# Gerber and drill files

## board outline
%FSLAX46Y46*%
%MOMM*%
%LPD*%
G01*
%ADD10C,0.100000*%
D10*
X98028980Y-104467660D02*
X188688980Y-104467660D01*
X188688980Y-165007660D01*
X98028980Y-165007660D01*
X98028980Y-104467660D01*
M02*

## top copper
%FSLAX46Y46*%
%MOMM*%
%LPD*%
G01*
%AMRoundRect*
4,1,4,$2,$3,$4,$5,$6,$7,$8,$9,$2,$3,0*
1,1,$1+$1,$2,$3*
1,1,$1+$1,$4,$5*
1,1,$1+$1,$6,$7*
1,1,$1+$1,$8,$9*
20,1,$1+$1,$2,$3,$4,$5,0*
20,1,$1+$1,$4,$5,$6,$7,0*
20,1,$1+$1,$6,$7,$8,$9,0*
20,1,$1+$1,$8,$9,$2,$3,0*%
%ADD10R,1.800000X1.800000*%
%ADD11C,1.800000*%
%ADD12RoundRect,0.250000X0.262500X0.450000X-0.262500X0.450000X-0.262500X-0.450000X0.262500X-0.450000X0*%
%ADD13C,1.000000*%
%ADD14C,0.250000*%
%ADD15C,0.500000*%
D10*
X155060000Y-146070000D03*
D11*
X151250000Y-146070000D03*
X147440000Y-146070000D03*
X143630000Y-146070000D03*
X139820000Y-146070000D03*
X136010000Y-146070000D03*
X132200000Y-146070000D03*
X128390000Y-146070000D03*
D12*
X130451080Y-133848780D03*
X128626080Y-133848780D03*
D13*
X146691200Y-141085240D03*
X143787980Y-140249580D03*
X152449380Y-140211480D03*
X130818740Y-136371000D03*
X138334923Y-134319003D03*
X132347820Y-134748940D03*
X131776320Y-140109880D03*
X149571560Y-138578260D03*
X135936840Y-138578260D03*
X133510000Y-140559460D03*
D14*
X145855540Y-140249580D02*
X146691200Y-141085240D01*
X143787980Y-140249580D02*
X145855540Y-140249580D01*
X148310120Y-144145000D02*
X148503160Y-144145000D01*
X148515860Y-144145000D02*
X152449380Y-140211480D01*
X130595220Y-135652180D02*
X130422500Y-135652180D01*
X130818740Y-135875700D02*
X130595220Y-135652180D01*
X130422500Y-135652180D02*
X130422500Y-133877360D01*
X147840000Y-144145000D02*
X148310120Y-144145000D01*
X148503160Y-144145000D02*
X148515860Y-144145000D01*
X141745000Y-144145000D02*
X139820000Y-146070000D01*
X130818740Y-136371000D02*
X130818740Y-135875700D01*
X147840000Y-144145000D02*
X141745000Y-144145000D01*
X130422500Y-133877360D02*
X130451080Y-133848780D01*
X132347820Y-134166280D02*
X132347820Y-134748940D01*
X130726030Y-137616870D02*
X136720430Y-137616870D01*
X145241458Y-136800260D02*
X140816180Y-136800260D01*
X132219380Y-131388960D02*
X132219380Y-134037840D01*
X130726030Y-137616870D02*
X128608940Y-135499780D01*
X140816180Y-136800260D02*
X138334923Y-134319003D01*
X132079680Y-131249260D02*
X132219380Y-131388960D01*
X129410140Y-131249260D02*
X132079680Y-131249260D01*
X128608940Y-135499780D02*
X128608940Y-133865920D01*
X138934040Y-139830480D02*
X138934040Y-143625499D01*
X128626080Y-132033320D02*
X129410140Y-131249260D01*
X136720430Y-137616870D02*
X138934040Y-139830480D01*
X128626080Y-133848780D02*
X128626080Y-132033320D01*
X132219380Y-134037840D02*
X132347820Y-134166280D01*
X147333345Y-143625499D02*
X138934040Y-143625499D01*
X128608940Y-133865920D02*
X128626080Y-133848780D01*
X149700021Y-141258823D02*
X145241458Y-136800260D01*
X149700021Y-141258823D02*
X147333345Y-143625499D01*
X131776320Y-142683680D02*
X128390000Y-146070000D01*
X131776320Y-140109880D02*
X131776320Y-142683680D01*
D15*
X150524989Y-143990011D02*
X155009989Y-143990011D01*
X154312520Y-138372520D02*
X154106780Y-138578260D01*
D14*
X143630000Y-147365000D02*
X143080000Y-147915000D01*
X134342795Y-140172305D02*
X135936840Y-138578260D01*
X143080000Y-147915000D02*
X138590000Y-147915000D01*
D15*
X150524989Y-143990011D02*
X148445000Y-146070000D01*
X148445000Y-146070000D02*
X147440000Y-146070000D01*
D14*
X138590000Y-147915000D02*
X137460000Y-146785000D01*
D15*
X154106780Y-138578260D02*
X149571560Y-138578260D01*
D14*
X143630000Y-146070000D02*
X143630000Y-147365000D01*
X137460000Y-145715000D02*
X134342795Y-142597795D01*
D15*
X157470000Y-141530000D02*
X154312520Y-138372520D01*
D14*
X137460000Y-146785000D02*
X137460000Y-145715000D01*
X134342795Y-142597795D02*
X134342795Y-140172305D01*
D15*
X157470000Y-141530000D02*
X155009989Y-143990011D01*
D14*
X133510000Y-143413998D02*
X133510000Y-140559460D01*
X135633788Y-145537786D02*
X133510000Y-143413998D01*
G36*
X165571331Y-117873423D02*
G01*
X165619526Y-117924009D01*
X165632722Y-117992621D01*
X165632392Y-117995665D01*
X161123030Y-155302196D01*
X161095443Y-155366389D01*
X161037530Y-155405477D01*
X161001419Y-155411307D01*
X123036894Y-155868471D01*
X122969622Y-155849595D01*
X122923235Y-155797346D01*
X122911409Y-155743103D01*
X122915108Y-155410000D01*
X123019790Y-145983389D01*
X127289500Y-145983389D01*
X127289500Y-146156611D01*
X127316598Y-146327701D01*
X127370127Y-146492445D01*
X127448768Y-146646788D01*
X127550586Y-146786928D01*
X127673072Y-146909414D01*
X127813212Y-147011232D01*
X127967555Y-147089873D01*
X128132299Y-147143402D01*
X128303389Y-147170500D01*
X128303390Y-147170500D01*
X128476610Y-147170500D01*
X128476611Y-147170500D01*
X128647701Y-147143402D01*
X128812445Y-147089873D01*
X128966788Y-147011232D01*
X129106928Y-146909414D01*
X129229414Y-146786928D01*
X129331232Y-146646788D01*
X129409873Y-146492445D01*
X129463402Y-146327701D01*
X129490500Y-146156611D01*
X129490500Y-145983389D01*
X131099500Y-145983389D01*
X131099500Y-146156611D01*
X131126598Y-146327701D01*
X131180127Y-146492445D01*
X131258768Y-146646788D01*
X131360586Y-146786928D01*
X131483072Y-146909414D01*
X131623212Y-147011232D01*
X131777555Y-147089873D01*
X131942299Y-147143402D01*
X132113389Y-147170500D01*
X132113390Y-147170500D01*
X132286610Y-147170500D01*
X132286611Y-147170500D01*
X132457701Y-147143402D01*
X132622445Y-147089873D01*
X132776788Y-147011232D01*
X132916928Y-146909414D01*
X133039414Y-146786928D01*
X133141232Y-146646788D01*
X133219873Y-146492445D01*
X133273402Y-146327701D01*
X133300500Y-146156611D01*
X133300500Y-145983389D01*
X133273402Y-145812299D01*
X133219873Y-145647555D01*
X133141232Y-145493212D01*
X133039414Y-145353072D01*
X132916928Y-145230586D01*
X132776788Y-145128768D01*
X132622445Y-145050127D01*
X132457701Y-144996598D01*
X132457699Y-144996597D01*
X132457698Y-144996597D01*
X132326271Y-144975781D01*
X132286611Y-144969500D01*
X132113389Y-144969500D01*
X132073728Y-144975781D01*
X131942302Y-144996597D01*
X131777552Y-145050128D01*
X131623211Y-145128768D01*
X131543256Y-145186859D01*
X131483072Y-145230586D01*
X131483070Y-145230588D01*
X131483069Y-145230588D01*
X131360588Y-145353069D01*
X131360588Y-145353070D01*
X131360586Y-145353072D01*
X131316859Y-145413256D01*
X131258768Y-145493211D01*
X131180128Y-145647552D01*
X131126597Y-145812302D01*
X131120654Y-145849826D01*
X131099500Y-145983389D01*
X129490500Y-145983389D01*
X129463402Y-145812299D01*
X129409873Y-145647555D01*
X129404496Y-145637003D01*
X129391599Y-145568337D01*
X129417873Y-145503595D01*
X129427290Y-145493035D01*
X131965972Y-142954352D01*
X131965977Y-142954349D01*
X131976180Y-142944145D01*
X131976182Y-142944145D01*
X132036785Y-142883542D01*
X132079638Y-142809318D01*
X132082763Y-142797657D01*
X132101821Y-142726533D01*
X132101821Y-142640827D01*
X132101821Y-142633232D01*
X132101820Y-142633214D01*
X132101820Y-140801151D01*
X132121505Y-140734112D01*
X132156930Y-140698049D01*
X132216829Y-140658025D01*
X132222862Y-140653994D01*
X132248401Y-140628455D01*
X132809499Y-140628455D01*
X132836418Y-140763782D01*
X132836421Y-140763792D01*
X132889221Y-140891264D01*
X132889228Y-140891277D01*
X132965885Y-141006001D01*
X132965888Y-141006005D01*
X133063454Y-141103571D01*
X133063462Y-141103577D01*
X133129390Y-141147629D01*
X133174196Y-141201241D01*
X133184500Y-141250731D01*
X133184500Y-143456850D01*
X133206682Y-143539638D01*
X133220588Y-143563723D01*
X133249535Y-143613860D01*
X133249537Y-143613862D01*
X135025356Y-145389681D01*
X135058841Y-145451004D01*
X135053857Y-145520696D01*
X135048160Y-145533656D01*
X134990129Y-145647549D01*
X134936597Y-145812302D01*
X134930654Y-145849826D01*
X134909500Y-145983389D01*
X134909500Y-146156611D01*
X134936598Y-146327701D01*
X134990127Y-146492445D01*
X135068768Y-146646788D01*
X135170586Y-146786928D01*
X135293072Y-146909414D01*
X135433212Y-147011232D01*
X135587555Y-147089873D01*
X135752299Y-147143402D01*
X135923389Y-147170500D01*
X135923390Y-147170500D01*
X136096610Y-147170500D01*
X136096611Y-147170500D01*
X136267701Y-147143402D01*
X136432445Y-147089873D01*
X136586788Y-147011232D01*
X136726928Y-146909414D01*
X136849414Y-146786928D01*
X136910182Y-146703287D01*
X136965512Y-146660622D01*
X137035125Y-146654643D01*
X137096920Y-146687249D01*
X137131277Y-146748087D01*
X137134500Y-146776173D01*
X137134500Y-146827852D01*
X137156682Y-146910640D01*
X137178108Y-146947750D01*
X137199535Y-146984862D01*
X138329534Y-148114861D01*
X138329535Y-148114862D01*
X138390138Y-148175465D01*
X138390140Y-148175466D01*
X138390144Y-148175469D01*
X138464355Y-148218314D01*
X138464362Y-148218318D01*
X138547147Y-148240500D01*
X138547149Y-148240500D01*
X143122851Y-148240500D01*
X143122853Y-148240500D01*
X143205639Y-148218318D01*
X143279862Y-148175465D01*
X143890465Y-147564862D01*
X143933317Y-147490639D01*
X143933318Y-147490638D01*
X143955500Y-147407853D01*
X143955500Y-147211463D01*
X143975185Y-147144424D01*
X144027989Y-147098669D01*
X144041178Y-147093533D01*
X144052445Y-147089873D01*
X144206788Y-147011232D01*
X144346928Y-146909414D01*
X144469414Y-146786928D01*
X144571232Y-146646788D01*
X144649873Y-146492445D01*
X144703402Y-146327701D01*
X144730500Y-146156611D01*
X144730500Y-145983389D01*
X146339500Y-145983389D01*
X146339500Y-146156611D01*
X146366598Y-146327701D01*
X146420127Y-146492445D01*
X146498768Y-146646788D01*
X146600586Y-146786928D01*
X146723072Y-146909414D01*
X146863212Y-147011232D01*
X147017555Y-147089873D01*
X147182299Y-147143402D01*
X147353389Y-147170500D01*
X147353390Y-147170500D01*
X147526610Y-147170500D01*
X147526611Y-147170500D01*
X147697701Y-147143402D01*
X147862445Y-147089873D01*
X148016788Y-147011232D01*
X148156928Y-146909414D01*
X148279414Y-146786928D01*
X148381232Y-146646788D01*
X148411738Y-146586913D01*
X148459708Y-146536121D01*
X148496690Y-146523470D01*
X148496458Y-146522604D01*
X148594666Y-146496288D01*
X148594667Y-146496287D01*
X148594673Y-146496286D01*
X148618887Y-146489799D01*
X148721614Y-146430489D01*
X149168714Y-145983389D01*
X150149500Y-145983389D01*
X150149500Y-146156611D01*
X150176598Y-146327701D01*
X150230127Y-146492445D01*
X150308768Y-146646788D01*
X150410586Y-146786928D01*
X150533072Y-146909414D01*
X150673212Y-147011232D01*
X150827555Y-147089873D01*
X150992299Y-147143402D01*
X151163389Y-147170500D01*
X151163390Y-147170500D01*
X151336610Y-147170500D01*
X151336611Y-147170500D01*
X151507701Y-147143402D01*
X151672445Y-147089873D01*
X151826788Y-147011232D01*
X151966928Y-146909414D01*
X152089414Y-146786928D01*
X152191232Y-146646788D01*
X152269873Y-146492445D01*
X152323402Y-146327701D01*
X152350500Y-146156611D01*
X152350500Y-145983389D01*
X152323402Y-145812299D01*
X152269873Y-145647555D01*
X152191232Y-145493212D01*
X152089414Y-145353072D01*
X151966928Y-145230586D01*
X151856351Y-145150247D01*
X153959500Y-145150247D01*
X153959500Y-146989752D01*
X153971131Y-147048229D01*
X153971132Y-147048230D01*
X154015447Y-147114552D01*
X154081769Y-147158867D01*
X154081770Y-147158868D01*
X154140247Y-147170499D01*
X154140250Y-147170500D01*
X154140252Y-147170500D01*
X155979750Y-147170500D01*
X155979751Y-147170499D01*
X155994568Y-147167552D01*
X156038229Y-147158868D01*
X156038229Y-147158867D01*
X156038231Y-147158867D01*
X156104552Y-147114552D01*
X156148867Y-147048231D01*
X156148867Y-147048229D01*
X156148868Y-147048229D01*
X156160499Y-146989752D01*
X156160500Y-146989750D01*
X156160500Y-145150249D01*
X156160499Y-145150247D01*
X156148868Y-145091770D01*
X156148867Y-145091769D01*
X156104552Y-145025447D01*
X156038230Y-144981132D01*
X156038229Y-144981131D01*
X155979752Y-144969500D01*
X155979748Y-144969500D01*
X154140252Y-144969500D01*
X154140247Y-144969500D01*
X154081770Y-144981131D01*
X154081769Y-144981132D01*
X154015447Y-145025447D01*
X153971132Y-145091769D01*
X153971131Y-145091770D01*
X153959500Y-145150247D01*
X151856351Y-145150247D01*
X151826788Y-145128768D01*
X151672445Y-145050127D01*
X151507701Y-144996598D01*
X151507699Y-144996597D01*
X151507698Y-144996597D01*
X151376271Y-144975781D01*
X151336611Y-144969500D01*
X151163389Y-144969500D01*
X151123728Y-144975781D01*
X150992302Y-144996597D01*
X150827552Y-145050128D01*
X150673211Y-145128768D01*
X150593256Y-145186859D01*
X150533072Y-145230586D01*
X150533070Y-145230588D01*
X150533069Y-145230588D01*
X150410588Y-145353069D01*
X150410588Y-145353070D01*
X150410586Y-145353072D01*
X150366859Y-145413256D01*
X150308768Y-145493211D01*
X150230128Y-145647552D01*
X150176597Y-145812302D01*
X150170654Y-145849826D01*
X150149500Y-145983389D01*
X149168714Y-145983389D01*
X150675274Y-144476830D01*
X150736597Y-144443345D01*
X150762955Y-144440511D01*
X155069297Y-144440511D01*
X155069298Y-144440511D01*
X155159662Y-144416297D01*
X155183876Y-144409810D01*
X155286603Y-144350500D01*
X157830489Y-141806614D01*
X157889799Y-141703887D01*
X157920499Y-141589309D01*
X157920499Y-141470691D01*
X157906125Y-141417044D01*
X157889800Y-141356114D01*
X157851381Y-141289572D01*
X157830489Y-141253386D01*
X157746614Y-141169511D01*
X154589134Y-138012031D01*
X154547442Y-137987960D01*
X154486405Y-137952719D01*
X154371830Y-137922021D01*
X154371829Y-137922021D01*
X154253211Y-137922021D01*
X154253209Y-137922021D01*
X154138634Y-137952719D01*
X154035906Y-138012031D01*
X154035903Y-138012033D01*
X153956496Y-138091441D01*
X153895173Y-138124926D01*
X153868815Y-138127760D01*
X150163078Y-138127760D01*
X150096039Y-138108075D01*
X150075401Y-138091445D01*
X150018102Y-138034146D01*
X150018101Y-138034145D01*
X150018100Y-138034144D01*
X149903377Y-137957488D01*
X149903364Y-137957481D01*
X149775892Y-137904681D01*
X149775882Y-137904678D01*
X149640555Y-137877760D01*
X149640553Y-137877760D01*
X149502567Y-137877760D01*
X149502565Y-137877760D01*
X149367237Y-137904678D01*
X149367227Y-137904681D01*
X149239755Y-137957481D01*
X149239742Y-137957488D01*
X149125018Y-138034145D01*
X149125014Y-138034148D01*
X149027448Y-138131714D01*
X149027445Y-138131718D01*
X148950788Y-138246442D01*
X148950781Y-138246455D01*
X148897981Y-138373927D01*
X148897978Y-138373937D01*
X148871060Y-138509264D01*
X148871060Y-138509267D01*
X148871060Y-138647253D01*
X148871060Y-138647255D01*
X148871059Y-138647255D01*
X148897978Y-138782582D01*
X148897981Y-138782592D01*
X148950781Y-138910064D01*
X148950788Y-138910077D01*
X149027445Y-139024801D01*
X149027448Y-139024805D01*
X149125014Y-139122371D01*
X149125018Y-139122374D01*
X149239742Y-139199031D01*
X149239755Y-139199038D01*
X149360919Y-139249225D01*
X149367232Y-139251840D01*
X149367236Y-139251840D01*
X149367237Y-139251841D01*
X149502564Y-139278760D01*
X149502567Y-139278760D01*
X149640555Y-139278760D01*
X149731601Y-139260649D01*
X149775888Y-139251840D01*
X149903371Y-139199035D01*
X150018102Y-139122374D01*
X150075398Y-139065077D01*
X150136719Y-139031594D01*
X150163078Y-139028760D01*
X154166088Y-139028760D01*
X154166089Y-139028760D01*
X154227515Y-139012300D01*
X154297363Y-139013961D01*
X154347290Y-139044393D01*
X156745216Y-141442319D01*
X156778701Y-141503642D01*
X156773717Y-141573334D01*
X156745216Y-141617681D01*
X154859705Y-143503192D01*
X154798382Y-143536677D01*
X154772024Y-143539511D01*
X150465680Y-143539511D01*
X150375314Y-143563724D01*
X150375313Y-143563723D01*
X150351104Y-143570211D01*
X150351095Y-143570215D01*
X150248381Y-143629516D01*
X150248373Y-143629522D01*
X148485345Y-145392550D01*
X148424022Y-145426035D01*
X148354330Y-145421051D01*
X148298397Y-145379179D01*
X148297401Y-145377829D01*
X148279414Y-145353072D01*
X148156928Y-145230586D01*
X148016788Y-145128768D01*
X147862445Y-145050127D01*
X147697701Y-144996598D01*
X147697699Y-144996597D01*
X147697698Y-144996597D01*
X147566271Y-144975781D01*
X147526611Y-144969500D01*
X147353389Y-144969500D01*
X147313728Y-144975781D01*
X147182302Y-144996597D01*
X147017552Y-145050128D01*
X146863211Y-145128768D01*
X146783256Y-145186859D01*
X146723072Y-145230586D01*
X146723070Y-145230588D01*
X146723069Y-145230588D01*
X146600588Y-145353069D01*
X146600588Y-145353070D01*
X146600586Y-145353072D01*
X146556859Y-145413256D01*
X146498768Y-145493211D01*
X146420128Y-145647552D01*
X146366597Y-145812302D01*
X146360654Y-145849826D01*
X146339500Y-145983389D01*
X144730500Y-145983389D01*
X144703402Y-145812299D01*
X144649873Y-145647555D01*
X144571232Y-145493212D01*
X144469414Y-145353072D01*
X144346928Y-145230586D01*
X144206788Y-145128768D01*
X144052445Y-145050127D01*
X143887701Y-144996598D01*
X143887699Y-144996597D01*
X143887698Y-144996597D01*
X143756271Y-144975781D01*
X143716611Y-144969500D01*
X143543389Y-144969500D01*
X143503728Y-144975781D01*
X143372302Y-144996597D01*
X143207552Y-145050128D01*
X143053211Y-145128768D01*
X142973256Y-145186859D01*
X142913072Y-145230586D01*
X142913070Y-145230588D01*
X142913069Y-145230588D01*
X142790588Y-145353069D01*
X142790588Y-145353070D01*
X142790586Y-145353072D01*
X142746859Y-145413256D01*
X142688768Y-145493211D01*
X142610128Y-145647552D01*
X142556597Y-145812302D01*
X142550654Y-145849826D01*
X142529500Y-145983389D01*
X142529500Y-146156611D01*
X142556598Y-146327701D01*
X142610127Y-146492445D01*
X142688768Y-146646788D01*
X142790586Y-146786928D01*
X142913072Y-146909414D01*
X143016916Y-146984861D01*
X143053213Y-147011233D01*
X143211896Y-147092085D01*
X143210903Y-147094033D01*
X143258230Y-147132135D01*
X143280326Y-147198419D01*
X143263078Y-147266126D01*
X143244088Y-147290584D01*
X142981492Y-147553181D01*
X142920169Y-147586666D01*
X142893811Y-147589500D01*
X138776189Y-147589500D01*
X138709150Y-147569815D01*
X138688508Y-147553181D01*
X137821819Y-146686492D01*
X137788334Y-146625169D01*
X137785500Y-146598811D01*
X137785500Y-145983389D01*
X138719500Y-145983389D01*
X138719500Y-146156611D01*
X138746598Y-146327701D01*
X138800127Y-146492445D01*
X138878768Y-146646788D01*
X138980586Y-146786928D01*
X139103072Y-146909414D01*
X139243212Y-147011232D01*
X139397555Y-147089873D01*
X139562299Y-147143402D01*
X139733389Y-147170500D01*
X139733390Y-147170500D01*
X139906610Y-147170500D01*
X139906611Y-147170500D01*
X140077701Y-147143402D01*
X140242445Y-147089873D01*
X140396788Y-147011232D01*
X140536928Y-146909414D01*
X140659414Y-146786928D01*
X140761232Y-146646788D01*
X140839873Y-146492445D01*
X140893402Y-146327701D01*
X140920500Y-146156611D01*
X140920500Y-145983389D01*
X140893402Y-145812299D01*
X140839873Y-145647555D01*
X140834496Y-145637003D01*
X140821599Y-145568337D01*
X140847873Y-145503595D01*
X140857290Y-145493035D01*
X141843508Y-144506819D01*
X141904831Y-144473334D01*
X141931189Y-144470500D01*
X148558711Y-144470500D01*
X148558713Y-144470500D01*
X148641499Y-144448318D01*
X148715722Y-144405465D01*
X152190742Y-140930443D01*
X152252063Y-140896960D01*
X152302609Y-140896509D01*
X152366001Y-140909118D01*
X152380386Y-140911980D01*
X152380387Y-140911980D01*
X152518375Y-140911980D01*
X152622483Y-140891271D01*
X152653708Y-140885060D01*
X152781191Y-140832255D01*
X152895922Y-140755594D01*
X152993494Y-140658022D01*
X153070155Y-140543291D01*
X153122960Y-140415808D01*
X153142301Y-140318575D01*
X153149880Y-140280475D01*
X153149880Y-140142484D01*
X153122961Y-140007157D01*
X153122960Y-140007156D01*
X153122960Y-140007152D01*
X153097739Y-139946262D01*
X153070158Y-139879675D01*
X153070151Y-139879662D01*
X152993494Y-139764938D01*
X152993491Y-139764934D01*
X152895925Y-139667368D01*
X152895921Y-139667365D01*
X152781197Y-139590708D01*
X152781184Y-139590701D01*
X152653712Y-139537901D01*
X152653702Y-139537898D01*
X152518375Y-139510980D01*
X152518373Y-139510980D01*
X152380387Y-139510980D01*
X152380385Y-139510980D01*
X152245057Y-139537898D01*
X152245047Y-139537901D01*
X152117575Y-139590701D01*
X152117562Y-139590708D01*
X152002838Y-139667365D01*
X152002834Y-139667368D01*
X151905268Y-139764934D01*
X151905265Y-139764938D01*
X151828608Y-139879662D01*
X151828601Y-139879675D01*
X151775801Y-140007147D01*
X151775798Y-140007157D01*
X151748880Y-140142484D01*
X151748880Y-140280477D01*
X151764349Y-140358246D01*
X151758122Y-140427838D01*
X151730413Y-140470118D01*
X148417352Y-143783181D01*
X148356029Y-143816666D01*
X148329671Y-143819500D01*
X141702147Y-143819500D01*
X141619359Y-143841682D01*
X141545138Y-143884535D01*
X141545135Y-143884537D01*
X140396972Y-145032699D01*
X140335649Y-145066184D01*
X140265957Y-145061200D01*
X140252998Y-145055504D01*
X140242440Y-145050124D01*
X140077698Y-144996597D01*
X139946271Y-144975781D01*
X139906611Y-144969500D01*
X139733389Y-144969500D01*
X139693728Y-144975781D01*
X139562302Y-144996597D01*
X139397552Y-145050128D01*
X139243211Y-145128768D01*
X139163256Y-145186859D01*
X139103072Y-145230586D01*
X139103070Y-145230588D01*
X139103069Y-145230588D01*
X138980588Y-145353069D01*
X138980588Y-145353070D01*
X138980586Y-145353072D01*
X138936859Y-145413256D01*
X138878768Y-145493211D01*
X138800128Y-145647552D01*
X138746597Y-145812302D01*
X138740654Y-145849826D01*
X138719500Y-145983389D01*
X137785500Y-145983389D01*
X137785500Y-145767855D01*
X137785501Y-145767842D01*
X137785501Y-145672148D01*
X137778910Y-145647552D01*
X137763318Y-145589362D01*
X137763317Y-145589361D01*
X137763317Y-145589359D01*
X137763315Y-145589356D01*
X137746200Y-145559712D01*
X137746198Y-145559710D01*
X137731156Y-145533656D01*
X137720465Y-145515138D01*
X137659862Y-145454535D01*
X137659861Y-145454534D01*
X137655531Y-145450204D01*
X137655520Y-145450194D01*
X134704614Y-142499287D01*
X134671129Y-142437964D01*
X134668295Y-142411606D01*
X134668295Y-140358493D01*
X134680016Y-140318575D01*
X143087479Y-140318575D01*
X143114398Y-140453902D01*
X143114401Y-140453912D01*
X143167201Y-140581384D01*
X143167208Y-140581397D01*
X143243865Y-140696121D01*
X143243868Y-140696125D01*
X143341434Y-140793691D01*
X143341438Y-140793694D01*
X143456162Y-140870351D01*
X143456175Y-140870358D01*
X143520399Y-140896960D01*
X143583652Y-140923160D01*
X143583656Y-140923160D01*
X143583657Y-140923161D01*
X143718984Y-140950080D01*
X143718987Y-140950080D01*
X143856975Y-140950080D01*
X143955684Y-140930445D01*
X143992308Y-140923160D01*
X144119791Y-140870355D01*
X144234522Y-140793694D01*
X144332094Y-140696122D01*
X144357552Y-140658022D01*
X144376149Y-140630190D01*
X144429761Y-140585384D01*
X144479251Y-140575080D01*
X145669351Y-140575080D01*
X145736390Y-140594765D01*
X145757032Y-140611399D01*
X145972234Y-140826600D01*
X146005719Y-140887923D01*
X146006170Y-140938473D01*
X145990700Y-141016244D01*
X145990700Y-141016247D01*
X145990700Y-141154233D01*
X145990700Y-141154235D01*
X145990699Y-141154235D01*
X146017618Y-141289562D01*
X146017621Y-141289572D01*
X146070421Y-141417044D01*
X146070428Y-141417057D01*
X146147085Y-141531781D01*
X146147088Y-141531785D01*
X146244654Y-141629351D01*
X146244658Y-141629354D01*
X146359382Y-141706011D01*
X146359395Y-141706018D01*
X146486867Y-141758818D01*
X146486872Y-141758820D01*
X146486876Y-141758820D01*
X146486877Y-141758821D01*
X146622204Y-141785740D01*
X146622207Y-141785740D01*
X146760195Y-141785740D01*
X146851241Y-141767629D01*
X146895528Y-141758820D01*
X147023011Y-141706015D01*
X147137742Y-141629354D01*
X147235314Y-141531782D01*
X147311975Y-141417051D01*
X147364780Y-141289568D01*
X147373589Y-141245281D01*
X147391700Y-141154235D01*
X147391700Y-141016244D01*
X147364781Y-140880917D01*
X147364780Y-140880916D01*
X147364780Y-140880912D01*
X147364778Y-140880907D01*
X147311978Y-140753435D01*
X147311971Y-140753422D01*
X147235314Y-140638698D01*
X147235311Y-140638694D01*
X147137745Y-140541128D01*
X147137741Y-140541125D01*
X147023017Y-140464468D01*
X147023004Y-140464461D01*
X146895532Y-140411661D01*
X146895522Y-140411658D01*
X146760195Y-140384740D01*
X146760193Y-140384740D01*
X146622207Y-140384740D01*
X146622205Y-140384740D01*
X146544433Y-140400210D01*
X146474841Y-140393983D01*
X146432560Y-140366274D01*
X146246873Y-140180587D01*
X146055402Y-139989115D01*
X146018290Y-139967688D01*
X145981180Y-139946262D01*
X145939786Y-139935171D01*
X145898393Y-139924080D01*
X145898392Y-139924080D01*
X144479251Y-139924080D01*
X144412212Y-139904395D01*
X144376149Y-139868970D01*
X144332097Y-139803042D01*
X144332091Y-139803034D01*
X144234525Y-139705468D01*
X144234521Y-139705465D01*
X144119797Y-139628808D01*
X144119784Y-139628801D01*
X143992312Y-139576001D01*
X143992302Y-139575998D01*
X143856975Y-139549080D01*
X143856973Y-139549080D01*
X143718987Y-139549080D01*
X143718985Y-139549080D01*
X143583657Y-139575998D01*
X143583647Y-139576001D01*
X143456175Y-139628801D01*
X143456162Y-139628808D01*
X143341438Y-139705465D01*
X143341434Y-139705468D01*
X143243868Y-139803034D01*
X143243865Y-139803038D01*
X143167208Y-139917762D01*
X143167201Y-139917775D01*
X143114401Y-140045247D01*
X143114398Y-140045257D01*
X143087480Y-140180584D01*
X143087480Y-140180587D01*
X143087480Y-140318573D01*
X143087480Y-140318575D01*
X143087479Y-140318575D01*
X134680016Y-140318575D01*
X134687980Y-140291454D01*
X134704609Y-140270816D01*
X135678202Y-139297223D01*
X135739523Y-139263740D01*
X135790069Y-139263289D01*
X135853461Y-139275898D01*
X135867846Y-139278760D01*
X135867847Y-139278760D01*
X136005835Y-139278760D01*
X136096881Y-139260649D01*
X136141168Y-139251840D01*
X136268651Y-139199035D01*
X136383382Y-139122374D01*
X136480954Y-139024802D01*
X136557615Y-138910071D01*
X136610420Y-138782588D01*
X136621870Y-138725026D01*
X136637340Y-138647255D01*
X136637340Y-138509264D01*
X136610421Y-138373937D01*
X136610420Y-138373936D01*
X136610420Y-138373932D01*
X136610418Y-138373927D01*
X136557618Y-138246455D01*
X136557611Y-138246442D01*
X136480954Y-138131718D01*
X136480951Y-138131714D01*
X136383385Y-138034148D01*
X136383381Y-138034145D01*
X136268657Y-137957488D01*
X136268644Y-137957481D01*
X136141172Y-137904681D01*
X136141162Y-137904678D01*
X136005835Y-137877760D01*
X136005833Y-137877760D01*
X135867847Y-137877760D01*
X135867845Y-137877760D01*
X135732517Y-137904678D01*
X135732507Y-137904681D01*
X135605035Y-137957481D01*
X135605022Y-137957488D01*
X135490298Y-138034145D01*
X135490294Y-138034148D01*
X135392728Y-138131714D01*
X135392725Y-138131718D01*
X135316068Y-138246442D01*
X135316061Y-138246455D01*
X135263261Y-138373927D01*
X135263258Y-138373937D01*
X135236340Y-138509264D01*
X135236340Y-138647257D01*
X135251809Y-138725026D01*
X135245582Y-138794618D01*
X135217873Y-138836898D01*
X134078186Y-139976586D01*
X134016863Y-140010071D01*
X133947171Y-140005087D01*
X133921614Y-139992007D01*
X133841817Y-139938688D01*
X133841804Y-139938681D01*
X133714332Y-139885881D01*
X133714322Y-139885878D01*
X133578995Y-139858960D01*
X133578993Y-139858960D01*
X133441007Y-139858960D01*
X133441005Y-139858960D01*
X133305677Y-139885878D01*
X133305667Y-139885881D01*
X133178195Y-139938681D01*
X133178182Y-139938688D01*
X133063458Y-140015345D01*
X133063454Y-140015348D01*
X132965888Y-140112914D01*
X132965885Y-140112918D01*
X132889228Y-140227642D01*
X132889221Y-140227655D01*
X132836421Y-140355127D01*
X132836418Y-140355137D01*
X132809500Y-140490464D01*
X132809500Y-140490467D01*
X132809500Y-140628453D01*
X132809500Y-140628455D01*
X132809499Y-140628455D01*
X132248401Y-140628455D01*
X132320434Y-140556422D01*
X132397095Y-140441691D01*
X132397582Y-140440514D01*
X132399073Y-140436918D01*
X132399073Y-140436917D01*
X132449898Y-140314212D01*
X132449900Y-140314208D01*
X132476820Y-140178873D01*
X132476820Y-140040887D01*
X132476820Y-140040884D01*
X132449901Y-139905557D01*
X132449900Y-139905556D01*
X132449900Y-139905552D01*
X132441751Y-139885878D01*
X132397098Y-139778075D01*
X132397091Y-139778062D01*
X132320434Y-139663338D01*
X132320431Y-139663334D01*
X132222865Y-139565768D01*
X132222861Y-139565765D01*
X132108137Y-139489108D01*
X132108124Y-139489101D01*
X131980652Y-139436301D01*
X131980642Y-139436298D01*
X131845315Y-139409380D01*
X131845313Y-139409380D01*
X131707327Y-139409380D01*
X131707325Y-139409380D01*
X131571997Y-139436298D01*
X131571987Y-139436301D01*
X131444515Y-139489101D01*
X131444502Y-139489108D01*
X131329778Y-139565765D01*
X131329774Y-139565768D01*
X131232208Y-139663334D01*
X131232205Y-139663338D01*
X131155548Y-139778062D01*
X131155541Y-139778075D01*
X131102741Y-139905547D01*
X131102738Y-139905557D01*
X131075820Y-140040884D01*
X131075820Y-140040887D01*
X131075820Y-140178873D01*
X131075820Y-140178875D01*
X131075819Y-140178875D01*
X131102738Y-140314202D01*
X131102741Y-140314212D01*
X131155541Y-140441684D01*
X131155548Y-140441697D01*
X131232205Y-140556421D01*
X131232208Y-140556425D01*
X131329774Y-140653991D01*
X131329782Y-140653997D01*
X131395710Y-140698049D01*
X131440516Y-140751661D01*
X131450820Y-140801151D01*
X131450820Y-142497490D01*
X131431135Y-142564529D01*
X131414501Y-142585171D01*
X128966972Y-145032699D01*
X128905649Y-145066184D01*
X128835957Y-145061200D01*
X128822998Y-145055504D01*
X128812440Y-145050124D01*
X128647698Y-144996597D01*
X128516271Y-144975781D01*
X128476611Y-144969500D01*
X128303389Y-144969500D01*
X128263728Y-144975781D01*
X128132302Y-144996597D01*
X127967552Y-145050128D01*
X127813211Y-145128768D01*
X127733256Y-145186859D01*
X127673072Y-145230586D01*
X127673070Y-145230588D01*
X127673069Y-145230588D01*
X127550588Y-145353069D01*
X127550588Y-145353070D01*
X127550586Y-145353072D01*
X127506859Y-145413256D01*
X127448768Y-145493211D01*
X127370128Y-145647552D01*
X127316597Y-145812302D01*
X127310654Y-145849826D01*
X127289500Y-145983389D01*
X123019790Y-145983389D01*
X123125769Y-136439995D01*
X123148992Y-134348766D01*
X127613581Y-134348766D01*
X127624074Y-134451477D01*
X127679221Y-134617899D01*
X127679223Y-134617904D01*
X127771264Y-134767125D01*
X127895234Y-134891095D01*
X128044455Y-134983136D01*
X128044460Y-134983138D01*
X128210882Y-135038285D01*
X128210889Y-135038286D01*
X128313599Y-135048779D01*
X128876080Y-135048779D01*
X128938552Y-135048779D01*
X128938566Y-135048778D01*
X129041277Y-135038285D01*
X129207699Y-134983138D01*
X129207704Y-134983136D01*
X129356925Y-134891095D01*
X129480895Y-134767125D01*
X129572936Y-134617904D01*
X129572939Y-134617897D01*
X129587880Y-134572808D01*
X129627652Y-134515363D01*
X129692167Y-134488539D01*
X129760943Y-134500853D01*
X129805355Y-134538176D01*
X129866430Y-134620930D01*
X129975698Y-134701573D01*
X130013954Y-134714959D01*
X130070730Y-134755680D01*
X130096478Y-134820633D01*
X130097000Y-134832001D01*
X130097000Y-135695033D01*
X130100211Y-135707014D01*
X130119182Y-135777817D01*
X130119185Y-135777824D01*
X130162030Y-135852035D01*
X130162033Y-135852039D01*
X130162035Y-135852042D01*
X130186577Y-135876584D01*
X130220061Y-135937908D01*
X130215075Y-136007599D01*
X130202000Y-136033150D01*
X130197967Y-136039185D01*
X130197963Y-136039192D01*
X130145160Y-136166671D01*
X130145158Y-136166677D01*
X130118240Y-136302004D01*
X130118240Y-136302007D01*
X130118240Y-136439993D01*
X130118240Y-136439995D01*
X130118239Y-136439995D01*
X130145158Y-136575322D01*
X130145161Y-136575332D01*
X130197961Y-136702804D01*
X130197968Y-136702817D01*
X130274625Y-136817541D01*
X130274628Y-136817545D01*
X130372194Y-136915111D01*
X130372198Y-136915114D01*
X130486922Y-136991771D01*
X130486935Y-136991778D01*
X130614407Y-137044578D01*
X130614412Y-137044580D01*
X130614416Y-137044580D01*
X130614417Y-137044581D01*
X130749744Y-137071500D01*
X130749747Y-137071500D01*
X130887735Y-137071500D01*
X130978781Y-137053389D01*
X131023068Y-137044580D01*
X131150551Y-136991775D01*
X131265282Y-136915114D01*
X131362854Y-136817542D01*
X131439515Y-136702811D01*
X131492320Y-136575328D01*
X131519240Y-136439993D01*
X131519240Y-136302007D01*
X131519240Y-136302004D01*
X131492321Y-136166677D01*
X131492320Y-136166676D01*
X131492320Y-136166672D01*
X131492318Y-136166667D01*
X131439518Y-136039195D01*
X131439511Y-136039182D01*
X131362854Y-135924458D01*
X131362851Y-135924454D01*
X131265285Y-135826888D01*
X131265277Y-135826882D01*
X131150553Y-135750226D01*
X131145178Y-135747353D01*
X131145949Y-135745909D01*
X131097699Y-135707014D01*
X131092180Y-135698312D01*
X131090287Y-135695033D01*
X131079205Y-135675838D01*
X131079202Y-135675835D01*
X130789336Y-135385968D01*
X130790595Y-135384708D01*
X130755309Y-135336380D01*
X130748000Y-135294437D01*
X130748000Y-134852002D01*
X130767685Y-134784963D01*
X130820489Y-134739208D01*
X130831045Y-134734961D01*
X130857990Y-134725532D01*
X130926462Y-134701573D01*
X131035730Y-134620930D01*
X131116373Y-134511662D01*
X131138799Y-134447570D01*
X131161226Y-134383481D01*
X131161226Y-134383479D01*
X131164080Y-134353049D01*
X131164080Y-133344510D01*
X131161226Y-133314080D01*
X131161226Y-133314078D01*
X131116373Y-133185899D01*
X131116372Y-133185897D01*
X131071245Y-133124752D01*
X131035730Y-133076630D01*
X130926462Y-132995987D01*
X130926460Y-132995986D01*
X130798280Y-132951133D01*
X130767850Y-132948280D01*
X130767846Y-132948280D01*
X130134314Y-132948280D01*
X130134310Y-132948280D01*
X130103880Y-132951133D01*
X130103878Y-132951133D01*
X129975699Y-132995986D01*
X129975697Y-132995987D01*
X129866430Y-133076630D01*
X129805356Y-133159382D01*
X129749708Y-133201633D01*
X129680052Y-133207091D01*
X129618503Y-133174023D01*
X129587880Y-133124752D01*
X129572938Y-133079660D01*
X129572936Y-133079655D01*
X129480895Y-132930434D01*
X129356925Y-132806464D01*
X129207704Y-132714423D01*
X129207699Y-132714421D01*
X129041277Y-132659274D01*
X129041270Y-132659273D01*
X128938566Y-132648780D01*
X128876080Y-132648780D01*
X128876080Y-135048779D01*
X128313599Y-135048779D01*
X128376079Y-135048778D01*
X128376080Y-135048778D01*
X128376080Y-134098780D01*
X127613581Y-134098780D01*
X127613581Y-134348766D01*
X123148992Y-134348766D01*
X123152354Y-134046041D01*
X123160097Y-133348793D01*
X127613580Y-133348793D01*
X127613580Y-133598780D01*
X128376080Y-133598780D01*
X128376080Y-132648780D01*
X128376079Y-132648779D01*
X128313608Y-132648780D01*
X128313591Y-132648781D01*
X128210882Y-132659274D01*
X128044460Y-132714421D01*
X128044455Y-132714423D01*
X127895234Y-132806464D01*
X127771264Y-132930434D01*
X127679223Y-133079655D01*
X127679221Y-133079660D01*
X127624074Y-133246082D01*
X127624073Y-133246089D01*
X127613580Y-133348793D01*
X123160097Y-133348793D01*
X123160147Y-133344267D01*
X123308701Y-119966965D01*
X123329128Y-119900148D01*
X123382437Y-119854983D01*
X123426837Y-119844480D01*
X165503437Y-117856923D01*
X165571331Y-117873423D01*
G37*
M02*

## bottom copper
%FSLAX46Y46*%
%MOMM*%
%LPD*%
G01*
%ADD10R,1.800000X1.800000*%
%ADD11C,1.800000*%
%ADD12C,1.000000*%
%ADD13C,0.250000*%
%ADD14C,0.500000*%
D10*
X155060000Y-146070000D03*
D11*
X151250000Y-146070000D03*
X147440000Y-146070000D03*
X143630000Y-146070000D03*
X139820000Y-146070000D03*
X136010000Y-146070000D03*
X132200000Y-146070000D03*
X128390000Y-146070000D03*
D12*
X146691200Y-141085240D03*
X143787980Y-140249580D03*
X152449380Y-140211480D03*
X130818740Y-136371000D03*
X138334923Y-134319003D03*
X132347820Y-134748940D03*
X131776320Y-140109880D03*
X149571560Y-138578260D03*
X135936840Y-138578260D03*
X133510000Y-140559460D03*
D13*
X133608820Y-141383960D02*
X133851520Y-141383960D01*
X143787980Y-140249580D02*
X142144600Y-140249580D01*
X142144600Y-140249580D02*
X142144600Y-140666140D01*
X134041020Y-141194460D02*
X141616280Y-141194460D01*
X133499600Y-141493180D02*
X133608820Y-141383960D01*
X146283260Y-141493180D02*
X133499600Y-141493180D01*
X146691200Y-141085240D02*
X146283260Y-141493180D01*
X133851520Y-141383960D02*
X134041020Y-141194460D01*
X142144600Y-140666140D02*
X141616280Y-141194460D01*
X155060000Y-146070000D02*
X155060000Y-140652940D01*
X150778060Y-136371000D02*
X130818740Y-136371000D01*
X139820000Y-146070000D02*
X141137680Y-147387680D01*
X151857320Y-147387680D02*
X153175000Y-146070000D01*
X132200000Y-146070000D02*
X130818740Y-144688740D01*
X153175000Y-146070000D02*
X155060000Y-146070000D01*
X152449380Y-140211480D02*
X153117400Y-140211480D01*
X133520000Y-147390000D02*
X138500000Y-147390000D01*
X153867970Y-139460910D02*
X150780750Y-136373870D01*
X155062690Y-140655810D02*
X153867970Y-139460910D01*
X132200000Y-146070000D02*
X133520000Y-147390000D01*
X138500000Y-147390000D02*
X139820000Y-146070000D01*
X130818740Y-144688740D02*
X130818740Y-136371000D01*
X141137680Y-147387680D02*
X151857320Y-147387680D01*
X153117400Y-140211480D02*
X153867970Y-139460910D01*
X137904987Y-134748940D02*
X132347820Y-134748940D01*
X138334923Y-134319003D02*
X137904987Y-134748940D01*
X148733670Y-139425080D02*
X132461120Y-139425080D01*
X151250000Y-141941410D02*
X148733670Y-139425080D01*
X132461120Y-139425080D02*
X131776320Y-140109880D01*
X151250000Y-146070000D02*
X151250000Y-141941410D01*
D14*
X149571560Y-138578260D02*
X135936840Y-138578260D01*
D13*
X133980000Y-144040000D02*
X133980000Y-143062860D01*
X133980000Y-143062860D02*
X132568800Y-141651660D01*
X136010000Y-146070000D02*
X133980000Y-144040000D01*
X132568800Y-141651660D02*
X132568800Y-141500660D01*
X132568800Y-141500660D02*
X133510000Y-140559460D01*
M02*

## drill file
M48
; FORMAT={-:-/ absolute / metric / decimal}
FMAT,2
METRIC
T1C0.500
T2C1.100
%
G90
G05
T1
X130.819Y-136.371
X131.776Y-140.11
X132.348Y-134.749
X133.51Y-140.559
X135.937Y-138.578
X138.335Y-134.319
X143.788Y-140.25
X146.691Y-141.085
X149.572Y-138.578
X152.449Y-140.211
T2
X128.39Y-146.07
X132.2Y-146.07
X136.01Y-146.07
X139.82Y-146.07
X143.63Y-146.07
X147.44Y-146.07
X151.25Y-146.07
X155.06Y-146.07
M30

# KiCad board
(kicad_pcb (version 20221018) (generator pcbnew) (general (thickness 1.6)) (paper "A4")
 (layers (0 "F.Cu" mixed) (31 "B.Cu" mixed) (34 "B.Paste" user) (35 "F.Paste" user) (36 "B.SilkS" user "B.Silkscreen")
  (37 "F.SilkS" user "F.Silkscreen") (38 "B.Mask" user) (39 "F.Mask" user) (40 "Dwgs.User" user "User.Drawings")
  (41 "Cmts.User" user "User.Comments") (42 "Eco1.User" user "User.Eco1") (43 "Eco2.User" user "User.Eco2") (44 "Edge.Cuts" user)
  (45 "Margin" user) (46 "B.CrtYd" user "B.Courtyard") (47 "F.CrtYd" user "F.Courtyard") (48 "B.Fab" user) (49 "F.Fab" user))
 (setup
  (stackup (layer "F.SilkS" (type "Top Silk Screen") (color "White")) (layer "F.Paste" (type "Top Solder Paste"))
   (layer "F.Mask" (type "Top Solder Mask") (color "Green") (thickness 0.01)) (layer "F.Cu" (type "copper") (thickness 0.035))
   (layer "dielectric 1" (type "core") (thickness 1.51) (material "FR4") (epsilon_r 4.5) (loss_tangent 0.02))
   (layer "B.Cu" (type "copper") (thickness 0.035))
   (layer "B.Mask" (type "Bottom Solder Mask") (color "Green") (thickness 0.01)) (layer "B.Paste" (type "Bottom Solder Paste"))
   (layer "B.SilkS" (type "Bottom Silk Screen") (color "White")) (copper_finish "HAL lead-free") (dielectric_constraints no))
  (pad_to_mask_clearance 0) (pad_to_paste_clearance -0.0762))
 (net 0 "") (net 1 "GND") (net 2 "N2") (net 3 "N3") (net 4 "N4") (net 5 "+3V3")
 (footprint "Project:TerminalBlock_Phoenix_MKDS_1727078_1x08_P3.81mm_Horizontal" (layer "F.Cu") (at 155.06 146.07 180)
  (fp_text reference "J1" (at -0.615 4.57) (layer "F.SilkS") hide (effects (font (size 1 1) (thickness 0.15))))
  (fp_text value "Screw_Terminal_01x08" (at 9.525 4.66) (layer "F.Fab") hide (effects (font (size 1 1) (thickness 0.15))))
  (pad "1" thru_hole rect (at 0 0 180) (size 1.8 1.8) (drill 1.1) (layers "*.Cu" "*.Mask") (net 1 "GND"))
  (pad "2" thru_hole circle (at 3.81 0 180) (size 1.8 1.8) (drill 1.1) (layers "*.Cu" "*.Mask") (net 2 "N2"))
  (pad "3" thru_hole circle (at 7.62 0 180) (size 1.8 1.8) (drill 1.1) (layers "*.Cu" "*.Mask") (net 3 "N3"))
  (pad "4" thru_hole circle (at 11.43 0 180) (size 1.8 1.8) (drill 1.1) (layers "*.Cu" "*.Mask") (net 3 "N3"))
  (pad "5" thru_hole circle (at 15.24 0 180) (size 1.8 1.8) (drill 1.1) (layers "*.Cu" "*.Mask") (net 1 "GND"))
  (pad "6" thru_hole circle (at 19.05 0 270) (size 1.8 1.8) (drill 1.1) (layers "*.Cu" "*.Mask") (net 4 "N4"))
  (pad "7" thru_hole circle (at 22.86 0 180) (size 1.8 1.8) (drill 1.1) (layers "*.Cu" "*.Mask") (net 1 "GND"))
  (pad "8" thru_hole circle (at 26.67 0 270) (size 1.8 1.8) (drill 1.1) (layers "*.Cu" "*.Mask") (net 2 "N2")))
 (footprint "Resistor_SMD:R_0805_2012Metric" (layer "F.Cu") (at 129.53858 133.84878 180)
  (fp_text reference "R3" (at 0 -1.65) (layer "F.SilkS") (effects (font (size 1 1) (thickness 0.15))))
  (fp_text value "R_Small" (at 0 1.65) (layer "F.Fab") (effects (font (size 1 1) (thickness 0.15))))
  (pad "1" smd roundrect (at -0.9125 0 180) (size 1.025 1.4) (layers "F.Cu" "F.Paste" "F.Mask") (roundrect_rratio 0.243902) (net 1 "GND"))
  (pad "2" smd roundrect (at 0.9125 0 180) (size 1.025 1.4) (layers "F.Cu" "F.Paste" "F.Mask") (roundrect_rratio 0.243902) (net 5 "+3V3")))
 (gr_rect (start 98.02898 104.46766) (end 188.68898 165.00766) (stroke (width 0.1) (type solid)) (fill none) (layer "Edge.Cuts"))
 (segment (start 145.85554 140.24958) (end 146.6912 141.08524) (width 0.25) (layer "F.Cu") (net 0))
 (segment (start 143.78798 140.24958) (end 145.85554 140.24958) (width 0.25) (layer "F.Cu") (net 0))
 (via (at 146.6912 141.08524) (size 1) (drill 0.5) (layers "F.Cu" "B.Cu") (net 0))
 (via (at 143.78798 140.24958) (size 1) (drill 0.5) (layers "F.Cu" "B.Cu") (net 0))
 (segment (start 133.60882 141.38396) (end 133.85152 141.38396) (width 0.25) (layer "B.Cu") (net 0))
 (segment locked (start 143.78798 140.24958) (end 142.1446 140.24958) (width 0.25) (layer "B.Cu") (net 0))
 (segment (start 142.1446 140.24958) (end 142.1446 140.66614) (width 0.25) (layer "B.Cu") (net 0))
 (segment (start 134.04102 141.19446) (end 141.61628 141.19446) (width 0.25) (layer "B.Cu") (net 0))
 (segment (start 133.4996 141.49318) (end 133.60882 141.38396) (width 0.25) (layer "B.Cu") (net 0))
 (segment (start 146.28326 141.49318) (end 133.4996 141.49318) (width 0.25) (layer "B.Cu") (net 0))
 (segment (start 146.6912 141.08524) (end 146.28326 141.49318) (width 0.25) (layer "B.Cu") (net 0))
 (segment (start 133.85152 141.38396) (end 134.04102 141.19446) (width 0.25) (layer "B.Cu") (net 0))
 (segment (start 142.1446 140.66614) (end 141.61628 141.19446) (width 0.25) (layer "B.Cu") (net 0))
 (segment (start 148.31012 144.145) (end 148.50316 144.145) (width 0.25) (layer "F.Cu") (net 1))
 (segment (start 148.51586 144.145) (end 152.44938 140.21148) (width 0.25) (layer "F.Cu") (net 1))
 (segment (start 130.59522 135.65218) (end 130.4225 135.65218) (width 0.25) (layer "F.Cu") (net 1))
 (segment (start 130.81874 135.8757) (end 130.59522 135.65218) (width 0.25) (layer "F.Cu") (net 1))
 (segment (start 130.4225 135.65218) (end 130.4225 133.87736) (width 0.25) (layer "F.Cu") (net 1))
 (segment (start 147.84 144.145) (end 148.31012 144.145) (width 0.25) (layer "F.Cu") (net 1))
 (segment (start 148.50316 144.145) (end 148.51586 144.145) (width 0.25) (layer "F.Cu") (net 1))
 (segment (start 141.745 144.145) (end 139.82 146.07) (width 0.25) (layer "F.Cu") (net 1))
 (segment (start 130.81874 136.371) (end 130.81874 135.8757) (width 0.25) (layer "F.Cu") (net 1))
 (segment (start 147.84 144.145) (end 141.745 144.145) (width 0.25) (layer "F.Cu") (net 1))
 (segment (start 130.4225 133.87736) (end 130.45108 133.84878) (width 0.25) (layer "F.Cu") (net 1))
 (via (at 152.44938 140.21148) (size 1) (drill 0.5) (layers "F.Cu" "B.Cu") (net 1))
 (via (at 130.81874 136.371) (size 1) (drill 0.5) (layers "F.Cu" "B.Cu") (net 1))
 (segment (start 155.06 146.07) (end 155.06 140.65294) (width 0.25) (layer "B.Cu") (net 1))
 (segment (start 150.77806 136.371) (end 130.81874 136.371) (width 0.25) (layer "B.Cu") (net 1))
 (segment (start 139.82 146.07) (end 141.13768 147.38768) (width 0.25) (layer "B.Cu") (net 1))
 (segment (start 151.85732 147.38768) (end 153.175 146.07) (width 0.25) (layer "B.Cu") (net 1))
 (segment (start 132.2 146.07) (end 130.81874 144.68874) (width 0.25) (layer "B.Cu") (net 1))
 (segment (start 153.175 146.07) (end 155.06 146.07) (width 0.25) (layer "B.Cu") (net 1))
 (segment (start 152.44938 140.21148) (end 153.1174 140.21148) (width 0.25) (layer "B.Cu") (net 1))
 (segment (start 133.52 147.39) (end 138.5 147.39) (width 0.25) (layer "B.Cu") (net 1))
 (segment (start 153.86797 139.46091) (end 150.78075 136.37387) (width 0.25) (layer "B.Cu") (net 1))
 (segment (start 155.06269 140.65581) (end 153.86797 139.46091) (width 0.25) (layer "B.Cu") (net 1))
 (segment (start 132.2 146.07) (end 133.52 147.39) (width 0.25) (layer "B.Cu") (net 1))
 (segment (start 138.5 147.39) (end 139.82 146.07) (width 0.25) (layer "B.Cu") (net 1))
 (segment (start 130.81874 144.68874) (end 130.81874 136.371) (width 0.25) (layer "B.Cu") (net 1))
 (segment (start 141.13768 147.38768) (end 151.85732 147.38768) (width 0.25) (layer "B.Cu") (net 1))
 (segment (start 153.1174 140.21148) (end 153.86797 139.46091) (width 0.25) (layer "B.Cu") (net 1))
 (segment (start 132.34782 134.16628) (end 132.34782 134.74894) (width 0.25) (layer "F.Cu") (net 5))
 (segment (start 130.72603 137.61687) (end 136.72043 137.61687) (width 0.25) (layer "F.Cu") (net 5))
 (segment (start 145.241458 136.80026) (end 140.81618 136.80026) (width 0.25) (layer "F.Cu") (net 5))
 (segment (start 132.21938 131.38896) (end 132.21938 134.03784) (width 0.25) (layer "F.Cu") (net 5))
 (segment (start 130.72603 137.61687) (end 128.60894 135.49978) (width 0.25) (layer "F.Cu") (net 5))
 (segment (start 140.81618 136.80026) (end 138.334923 134.319003) (width 0.25) (layer "F.Cu") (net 5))
 (segment (start 132.07968 131.24926) (end 132.21938 131.38896) (width 0.25) (layer "F.Cu") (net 5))
 (segment (start 129.41014 131.24926) (end 132.07968 131.24926) (width 0.25) (layer "F.Cu") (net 5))
 (segment (start 128.60894 135.49978) (end 128.60894 133.86592) (width 0.25) (layer "F.Cu") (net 5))
 (segment (start 138.93404 139.83048) (end 138.93404 143.625499) (width 0.25) (layer "F.Cu") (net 5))
 (segment (start 128.62608 132.03332) (end 129.41014 131.24926) (width 0.25) (layer "F.Cu") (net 5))
 (segment (start 136.72043 137.61687) (end 138.93404 139.83048) (width 0.25) (layer "F.Cu") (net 5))
 (segment (start 128.62608 133.84878) (end 128.62608 132.03332) (width 0.25) (layer "F.Cu") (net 5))
 (segment (start 132.21938 134.03784) (end 132.34782 134.16628) (width 0.25) (layer "F.Cu") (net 5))
 (segment (start 147.333345 143.625499) (end 138.93404 143.625499) (width 0.25) (layer "F.Cu") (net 5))
 (segment (start 128.60894 133.86592) (end 128.62608 133.84878) (width 0.25) (layer "F.Cu") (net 5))
 (segment (start 149.700021 141.258823) (end 145.241458 136.80026) (width 0.25) (layer "F.Cu") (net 5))
 (segment (start 149.700021 141.258823) (end 147.333345 143.625499) (width 0.25) (layer "F.Cu") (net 5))
 (via (at 138.334923 134.319003) (size 1) (drill 0.5) (layers "F.Cu" "B.Cu") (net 5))
 (via (at 132.34782 134.74894) (size 1) (drill 0.5) (layers "F.Cu" "B.Cu") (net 5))
 (segment (start 137.904987 134.74894) (end 132.34782 134.74894) (width 0.25) (layer "B.Cu") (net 5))
 (segment (start 138.334923 134.319003) (end 137.904987 134.74894) (width 0.25) (layer "B.Cu") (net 5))
 (segment (start 131.77632 142.68368) (end 128.39 146.07) (width 0.25) (layer "F.Cu") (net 2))
 (segment (start 131.77632 140.10988) (end 131.77632 142.68368) (width 0.25) (layer "F.Cu") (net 2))
 (via (at 131.77632 140.10988) (size 1) (drill 0.5) (layers "F.Cu" "B.Cu") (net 2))
 (segment (start 148.73367 139.42508) (end 132.46112 139.42508) (width 0.25) (layer "B.Cu") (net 2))
 (segment (start 151.25 141.94141) (end 148.73367 139.42508) (width 0.25) (layer "B.Cu") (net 2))
 (segment (start 132.46112 139.42508) (end 131.77632 140.10988) (width 0.25) (layer "B.Cu") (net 2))
 (segment (start 151.25 146.07) (end 151.25 141.94141) (width 0.25) (layer "B.Cu") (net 2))
 (segment (start 150.524989 143.990011) (end 155.009989 143.990011) (width 0.5) (layer "F.Cu") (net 3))
 (segment (start 154.31252 138.37252) (end 154.10678 138.57826) (width 0.5) (layer "F.Cu") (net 3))
 (segment (start 143.63 147.365) (end 143.08 147.915) (width 0.25) (layer "F.Cu") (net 3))
 (segment (start 134.342795 140.172305) (end 135.93684 138.57826) (width 0.25) (layer "F.Cu") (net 3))
 (segment (start 143.08 147.915) (end 138.59 147.915) (width 0.25) (layer "F.Cu") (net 3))
 (segment (start 150.524989 143.990011) (end 148.445 146.07) (width 0.5) (layer "F.Cu") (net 3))
 (segment (start 148.445 146.07) (end 147.44 146.07) (width 0.5) (layer "F.Cu") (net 3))
 (segment (start 138.59 147.915) (end 137.46 146.785) (width 0.25) (layer "F.Cu") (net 3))
 (segment (start 154.10678 138.57826) (end 149.57156 138.57826) (width 0.5) (layer "F.Cu") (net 3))
 (segment (start 143.63 146.07) (end 143.63 147.365) (width 0.25) (layer "F.Cu") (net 3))
 (segment (start 137.46 145.715) (end 134.342795 142.597795) (width 0.25) (layer "F.Cu") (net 3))
 (segment (start 157.47 141.53) (end 154.31252 138.37252) (width 0.5) (layer "F.Cu") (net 3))
 (segment (start 137.46 146.785) (end 137.46 145.715) (width 0.25) (layer "F.Cu") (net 3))
 (segment (start 134.342795 142.597795) (end 134.342795 140.172305) (width 0.25) (layer "F.Cu") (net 3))
 (segment (start 157.47 141.53) (end 155.009989 143.990011) (width 0.5) (layer "F.Cu") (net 3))
 (via (at 149.57156 138.57826) (size 1) (drill 0.5) (layers "F.Cu" "B.Cu") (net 3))
 (via (at 135.93684 138.57826) (size 1) (drill 0.5) (layers "F.Cu" "B.Cu") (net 3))
 (segment (start 149.57156 138.57826) (end 135.93684 138.57826) (width 0.5) (layer "B.Cu") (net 3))
 (segment (start 133.51 143.413998) (end 133.51 140.55946) (width 0.25) (layer "F.Cu") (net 4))
 (segment (start 135.633788 145.537786) (end 133.51 143.413998) (width 0.25) (layer "F.Cu") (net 4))
 (via (at 133.51 140.55946) (size 1) (drill 0.5) (layers "F.Cu" "B.Cu") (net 4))
 (segment (start 133.98 144.04) (end 133.98 143.06286) (width 0.25) (layer "B.Cu") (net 4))
 (segment (start 133.98 143.06286) (end 132.5688 141.65166) (width 0.25) (layer "B.Cu") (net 4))
 (segment (start 136.01 146.07) (end 133.98 144.04) (width 0.25) (layer "B.Cu") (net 4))
 (segment (start 132.5688 141.65166) (end 132.5688 141.50066) (width 0.25) (layer "B.Cu") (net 4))
 (segment (start 132.5688 141.50066) (end 133.51 140.55946) (width 0.25) (layer "B.Cu") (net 4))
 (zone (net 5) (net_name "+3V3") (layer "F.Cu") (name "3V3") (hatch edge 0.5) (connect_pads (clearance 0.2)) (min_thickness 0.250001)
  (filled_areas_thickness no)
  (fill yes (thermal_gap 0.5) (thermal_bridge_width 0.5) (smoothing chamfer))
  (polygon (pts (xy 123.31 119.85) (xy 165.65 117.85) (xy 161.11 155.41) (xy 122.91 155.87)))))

